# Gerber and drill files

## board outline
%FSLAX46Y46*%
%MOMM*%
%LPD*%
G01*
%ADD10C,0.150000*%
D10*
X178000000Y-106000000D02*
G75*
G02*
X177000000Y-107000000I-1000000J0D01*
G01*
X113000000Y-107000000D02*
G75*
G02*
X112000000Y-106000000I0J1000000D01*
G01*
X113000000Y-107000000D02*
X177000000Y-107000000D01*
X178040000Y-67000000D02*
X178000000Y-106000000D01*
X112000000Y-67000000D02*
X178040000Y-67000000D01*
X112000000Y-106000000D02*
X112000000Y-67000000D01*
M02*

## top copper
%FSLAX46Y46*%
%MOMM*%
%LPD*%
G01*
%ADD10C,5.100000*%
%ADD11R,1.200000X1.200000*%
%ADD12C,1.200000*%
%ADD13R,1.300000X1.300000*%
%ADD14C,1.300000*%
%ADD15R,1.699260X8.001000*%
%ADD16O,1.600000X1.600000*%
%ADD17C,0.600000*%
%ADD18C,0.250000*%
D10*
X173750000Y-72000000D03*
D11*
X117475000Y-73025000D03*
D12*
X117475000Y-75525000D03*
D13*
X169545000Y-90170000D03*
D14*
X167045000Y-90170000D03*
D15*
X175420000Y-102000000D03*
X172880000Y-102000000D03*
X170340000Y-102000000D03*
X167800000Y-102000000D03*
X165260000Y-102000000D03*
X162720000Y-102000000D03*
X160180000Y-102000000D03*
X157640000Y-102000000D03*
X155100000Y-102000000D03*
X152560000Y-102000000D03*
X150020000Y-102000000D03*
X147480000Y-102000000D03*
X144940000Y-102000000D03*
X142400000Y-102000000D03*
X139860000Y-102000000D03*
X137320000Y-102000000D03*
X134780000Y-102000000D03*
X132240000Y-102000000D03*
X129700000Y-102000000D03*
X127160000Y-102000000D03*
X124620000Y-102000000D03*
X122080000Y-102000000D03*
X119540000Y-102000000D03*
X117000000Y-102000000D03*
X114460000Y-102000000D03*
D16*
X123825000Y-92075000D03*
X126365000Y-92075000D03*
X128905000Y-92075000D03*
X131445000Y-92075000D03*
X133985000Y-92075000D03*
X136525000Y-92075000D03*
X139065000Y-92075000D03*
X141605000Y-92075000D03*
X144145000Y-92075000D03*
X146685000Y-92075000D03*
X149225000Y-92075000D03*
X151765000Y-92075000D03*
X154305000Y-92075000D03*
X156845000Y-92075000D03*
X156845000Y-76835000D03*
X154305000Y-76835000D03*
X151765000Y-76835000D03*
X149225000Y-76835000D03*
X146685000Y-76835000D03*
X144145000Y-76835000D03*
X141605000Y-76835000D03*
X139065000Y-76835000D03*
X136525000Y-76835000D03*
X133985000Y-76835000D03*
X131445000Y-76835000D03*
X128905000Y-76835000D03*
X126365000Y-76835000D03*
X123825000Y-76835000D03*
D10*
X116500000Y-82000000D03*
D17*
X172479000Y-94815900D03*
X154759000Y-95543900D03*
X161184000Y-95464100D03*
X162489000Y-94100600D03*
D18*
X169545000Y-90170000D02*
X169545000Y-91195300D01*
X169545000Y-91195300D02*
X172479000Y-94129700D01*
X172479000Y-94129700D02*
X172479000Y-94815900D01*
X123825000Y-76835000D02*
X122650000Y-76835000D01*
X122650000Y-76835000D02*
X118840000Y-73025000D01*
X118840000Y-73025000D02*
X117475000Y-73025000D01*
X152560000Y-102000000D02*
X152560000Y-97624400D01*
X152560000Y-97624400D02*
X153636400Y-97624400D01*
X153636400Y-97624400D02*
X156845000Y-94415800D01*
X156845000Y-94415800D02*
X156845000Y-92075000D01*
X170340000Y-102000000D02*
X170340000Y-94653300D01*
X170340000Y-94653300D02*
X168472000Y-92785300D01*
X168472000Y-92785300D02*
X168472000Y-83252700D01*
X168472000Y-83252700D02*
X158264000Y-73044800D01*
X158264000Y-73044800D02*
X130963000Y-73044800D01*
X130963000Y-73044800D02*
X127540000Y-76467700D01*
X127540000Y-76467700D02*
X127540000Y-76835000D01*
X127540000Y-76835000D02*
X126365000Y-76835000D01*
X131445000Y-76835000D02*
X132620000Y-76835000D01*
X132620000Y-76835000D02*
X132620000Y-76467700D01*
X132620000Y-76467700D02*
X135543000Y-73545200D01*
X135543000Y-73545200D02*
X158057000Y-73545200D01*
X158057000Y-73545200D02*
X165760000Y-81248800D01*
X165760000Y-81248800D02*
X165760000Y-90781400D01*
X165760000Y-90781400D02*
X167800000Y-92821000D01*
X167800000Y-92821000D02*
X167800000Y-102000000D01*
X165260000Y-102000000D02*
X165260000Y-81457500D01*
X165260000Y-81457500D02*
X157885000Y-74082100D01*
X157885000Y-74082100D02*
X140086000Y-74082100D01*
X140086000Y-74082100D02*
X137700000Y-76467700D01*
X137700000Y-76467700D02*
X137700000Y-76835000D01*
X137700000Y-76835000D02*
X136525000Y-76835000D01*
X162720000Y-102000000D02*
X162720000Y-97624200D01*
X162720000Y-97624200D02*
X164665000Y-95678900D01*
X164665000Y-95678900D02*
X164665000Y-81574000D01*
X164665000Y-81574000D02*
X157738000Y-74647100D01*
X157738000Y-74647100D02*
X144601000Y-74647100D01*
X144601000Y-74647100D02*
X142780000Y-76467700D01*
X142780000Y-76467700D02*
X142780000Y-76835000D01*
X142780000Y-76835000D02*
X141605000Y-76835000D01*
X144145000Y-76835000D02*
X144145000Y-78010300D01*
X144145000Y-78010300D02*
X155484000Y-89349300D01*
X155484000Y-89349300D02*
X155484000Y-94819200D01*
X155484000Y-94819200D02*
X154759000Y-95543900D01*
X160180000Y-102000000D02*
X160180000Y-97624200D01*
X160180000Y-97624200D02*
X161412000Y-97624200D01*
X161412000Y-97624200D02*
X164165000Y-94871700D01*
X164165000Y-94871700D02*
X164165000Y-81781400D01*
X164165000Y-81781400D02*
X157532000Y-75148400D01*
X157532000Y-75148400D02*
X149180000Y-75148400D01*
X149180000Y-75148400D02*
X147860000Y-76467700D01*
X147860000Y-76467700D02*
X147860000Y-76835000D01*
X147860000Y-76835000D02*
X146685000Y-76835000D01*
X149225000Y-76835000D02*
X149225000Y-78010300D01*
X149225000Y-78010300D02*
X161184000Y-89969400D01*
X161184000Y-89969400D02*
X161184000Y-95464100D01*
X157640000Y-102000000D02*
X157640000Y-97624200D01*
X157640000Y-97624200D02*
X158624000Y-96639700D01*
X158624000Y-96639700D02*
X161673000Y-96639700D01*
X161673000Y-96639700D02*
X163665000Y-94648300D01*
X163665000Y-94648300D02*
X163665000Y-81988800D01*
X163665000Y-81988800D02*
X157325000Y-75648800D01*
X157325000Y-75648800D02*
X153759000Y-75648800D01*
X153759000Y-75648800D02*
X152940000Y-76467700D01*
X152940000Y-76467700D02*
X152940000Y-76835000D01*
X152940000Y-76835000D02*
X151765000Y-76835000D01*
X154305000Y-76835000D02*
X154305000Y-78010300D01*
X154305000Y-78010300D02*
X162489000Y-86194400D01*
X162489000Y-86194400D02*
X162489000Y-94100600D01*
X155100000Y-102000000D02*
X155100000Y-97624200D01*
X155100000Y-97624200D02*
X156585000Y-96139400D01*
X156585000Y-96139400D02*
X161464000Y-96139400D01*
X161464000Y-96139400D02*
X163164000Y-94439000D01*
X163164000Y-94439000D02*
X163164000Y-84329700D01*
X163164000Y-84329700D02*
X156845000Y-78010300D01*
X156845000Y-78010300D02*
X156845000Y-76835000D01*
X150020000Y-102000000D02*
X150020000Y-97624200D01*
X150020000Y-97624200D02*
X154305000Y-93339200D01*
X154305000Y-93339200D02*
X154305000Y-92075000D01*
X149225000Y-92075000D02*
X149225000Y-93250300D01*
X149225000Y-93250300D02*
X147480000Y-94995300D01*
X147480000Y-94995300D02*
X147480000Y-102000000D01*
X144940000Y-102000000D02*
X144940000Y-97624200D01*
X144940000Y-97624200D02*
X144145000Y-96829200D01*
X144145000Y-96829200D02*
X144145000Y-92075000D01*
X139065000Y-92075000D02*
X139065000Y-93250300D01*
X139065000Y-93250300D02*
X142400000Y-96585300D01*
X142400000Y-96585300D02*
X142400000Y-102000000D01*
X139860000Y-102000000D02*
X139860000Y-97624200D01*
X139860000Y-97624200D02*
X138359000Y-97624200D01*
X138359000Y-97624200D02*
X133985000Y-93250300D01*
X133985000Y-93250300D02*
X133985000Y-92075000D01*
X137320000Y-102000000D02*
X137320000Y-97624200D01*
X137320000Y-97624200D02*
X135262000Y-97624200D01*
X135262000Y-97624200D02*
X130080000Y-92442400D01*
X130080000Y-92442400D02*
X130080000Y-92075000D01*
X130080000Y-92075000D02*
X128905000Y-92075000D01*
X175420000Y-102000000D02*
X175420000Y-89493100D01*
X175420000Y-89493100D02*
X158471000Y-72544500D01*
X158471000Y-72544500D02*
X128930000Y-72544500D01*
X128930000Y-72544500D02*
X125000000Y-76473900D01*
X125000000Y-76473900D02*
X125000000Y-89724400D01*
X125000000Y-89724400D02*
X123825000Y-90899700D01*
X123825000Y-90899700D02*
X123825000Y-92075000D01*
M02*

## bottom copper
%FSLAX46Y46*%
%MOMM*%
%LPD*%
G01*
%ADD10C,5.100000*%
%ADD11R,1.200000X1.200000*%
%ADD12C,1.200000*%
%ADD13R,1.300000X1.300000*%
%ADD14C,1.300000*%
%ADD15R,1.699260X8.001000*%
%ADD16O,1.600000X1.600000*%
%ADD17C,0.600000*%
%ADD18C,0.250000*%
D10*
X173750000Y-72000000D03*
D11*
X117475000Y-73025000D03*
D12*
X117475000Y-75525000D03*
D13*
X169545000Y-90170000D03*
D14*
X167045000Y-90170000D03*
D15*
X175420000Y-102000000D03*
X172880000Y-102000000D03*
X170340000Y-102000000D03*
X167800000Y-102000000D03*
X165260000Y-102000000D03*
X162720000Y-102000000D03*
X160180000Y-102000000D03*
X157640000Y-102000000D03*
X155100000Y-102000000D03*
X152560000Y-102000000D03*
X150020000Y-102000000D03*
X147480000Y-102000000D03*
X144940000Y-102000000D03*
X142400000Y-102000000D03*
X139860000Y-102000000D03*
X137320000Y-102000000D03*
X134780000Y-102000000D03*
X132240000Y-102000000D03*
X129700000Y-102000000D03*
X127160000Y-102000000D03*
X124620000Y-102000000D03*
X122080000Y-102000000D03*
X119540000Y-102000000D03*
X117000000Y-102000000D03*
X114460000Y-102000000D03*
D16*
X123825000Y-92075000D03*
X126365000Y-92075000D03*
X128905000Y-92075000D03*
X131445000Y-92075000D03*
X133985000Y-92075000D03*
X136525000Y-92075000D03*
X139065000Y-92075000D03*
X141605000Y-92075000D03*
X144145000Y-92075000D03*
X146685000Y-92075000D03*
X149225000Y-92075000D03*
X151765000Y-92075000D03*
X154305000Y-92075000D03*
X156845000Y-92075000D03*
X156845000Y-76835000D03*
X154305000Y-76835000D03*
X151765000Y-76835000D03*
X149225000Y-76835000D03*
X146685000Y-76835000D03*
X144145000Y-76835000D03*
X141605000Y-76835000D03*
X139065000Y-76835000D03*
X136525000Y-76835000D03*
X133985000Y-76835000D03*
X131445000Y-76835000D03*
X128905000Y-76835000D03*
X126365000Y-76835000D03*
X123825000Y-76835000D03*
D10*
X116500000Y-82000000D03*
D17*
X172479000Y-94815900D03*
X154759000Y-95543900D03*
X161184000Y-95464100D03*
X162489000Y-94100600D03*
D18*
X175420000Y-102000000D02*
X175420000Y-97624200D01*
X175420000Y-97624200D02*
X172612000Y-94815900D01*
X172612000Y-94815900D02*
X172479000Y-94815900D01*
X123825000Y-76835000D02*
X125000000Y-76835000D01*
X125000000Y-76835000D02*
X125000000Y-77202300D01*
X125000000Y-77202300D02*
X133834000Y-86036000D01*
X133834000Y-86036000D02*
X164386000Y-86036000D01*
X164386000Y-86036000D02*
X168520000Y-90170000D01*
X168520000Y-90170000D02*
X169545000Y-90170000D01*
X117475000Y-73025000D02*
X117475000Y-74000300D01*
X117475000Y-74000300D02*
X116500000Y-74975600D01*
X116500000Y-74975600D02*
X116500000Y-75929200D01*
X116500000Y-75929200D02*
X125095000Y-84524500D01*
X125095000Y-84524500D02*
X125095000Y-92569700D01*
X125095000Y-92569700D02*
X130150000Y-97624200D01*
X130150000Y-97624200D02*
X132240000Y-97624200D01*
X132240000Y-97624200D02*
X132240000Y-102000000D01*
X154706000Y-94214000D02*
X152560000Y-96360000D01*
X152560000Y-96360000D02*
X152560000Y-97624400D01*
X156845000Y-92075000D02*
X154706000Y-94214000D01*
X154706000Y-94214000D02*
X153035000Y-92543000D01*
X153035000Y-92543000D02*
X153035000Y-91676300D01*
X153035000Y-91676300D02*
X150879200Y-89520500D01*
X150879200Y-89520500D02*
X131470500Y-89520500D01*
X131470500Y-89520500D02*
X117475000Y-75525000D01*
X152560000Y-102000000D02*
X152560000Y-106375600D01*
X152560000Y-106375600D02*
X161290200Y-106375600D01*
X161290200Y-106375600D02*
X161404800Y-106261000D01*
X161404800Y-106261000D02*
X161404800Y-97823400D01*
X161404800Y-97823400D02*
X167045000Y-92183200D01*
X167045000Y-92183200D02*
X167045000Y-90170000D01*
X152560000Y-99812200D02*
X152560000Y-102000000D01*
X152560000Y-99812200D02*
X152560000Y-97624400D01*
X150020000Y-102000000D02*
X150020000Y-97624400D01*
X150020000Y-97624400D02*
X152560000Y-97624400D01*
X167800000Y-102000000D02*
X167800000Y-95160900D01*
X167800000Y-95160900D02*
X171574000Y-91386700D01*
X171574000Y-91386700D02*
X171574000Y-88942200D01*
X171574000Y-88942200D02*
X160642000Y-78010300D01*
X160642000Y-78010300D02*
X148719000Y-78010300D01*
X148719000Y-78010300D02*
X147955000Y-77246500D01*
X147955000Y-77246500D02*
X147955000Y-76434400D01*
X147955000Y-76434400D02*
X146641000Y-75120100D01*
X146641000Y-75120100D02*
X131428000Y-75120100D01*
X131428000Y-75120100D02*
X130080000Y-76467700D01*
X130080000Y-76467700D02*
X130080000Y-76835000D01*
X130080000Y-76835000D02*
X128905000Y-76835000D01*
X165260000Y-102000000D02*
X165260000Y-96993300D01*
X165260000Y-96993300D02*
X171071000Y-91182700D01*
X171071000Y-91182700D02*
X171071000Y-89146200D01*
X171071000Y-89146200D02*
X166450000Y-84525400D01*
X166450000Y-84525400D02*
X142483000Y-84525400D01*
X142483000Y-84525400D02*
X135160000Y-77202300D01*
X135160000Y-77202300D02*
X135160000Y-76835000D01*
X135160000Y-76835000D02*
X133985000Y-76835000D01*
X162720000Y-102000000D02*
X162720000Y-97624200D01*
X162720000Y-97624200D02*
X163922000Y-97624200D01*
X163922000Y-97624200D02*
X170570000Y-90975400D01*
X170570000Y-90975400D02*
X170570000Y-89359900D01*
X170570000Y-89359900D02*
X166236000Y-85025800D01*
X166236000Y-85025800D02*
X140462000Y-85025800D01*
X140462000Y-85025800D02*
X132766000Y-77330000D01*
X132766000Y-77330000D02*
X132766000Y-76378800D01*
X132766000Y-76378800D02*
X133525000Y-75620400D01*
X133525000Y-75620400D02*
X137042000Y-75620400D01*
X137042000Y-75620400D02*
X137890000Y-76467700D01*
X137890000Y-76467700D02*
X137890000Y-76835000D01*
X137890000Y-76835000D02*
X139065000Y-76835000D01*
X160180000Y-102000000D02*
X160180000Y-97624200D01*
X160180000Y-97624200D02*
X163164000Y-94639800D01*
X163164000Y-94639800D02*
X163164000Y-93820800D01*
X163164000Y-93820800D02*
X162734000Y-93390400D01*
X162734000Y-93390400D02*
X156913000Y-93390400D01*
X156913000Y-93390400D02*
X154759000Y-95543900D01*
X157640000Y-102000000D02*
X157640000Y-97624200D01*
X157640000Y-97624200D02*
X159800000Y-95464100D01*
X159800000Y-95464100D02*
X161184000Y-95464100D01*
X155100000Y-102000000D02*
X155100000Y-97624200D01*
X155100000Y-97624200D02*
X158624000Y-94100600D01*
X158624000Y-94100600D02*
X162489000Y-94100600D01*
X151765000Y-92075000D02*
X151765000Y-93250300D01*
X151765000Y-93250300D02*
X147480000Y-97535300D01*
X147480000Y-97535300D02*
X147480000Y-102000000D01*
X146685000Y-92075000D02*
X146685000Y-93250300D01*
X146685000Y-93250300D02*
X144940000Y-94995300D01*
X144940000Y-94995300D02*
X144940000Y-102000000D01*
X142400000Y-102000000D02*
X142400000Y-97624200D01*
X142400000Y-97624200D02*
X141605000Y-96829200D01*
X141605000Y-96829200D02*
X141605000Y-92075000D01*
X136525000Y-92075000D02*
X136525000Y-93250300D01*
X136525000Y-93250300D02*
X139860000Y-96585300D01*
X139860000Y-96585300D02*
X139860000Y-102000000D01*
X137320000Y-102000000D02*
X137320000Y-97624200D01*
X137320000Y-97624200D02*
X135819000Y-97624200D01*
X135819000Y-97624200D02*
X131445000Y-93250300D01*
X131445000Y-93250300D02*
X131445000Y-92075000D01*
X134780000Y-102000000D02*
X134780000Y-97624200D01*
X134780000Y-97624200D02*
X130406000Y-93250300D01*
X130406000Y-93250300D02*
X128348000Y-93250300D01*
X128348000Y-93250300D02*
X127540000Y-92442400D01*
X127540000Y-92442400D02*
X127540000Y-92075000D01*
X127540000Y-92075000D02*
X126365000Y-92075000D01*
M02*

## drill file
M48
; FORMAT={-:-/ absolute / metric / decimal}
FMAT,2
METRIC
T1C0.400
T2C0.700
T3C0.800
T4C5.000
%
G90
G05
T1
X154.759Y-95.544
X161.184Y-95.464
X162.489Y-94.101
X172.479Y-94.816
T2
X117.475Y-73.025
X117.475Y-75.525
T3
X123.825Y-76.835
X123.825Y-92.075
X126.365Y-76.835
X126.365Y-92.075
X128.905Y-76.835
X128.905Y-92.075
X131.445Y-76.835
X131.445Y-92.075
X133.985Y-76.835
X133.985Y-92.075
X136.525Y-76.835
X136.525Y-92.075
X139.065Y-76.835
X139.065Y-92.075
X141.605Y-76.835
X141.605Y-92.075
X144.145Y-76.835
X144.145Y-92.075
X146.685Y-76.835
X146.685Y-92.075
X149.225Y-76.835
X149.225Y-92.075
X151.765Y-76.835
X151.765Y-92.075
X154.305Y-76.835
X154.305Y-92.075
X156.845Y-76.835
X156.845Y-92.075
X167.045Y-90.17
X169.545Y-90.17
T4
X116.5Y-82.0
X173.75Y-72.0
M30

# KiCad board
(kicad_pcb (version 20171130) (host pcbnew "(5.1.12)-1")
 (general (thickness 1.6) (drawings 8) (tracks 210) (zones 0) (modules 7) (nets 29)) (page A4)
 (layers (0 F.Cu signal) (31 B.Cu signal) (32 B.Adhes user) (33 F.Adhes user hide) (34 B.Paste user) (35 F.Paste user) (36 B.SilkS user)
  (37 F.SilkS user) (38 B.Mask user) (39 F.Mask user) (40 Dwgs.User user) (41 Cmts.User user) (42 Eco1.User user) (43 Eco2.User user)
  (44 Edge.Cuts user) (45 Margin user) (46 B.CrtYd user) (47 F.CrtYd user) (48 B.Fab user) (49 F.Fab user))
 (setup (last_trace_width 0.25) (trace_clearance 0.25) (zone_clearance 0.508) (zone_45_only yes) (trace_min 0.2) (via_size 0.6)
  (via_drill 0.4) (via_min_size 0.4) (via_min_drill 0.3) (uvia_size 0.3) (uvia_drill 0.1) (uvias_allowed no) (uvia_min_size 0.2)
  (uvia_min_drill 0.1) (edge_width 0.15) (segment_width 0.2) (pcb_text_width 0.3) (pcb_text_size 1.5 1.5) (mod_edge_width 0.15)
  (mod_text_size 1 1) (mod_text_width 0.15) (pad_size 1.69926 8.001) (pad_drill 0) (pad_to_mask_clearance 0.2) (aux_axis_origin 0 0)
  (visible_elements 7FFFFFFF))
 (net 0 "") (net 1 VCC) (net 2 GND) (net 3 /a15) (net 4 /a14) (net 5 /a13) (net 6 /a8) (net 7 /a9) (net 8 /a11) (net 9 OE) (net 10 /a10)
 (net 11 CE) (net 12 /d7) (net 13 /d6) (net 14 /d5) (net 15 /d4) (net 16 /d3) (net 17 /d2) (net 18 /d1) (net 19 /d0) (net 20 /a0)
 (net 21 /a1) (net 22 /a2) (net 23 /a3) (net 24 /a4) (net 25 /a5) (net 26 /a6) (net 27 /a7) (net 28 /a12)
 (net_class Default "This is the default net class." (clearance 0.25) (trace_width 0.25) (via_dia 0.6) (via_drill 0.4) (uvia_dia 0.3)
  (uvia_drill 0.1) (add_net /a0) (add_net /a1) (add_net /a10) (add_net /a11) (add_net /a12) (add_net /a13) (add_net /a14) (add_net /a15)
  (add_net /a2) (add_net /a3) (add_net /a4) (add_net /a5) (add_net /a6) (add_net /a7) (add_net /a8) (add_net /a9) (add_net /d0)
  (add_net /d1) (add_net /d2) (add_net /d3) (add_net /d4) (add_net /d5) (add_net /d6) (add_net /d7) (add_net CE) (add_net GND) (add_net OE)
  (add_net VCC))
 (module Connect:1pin (layer F.Cu) (at 173.75 72)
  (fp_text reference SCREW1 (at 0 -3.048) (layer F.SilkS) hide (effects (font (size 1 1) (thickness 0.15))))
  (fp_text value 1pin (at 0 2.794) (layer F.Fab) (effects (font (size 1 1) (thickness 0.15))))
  (pad "" np_thru_hole circle (at 0 0) (size 5.1 5.1) (drill 5) (layers *.Cu)))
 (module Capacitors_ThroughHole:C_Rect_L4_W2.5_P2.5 (layer F.Cu) (at 117.475 73.025 270)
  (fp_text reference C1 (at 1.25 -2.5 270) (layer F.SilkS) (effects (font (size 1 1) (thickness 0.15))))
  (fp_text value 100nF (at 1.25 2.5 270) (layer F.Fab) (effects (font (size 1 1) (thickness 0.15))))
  (pad 1 thru_hole rect (at 0 0 270) (size 1.2 1.2) (drill 0.7) (layers *.Cu *.Mask F.SilkS) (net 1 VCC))
  (pad 2 thru_hole circle (at 2.5 0 270) (size 1.2 1.2) (drill 0.7) (layers *.Cu *.Mask F.SilkS) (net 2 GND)))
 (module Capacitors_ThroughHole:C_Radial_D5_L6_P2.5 (layer F.Cu) (at 169.545 90.17 180)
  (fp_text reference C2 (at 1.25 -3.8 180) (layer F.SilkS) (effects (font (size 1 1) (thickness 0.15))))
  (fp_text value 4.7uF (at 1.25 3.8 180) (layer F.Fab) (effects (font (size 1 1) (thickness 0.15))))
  (pad 1 thru_hole rect (at 0 0 180) (size 1.3 1.3) (drill 0.8) (layers *.Cu *.Mask F.SilkS) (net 1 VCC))
  (pad 2 thru_hole circle (at 2.5 0 180) (size 1.3 1.3) (drill 0.8) (layers *.Cu *.Mask F.SilkS) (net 2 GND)))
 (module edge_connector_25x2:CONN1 (layer F.Cu) (at 144.94 107.08)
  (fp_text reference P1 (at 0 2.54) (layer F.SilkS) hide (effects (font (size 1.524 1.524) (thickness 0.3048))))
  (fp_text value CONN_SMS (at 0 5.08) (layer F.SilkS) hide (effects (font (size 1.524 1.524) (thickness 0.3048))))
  (pad 1 connect rect (at 30.48 -5.08) (size 1.69926 8.001) (layers B.Cu B.Mask) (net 1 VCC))
  (pad 2 connect rect (at 30.48 -5.08) (size 1.69926 8.001) (layers F.Cu F.Mask) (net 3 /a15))
  (pad 3 connect rect (at 27.94 -5.08) (size 1.69926 8.001) (layers B.Cu B.Mask))
  (pad 4 connect rect (at 27.94 -5.08) (size 1.69926 8.001) (layers F.Cu F.Mask))
  (pad 5 connect rect (at 25.4 -5.08) (size 1.69926 8.001) (layers B.Cu B.Mask))
  (pad 6 connect rect (at 25.4 -5.08) (size 1.69926 8.001) (layers F.Cu F.Mask) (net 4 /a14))
  (pad 7 connect rect (at 22.86 -5.08) (size 1.69926 8.001) (layers B.Cu B.Mask) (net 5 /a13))
  (pad 8 connect rect (at 22.86 -5.08) (size 1.69926 8.001) (layers F.Cu F.Mask) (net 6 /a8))
  (pad 9 connect rect (at 20.32 -5.08) (size 1.69926 8.001) (layers B.Cu B.Mask) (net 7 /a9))
  (pad 10 connect rect (at 20.32 -5.08) (size 1.69926 8.001) (layers F.Cu F.Mask) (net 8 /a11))
  (pad 11 connect rect (at 17.78 -5.08) (size 1.69926 8.001) (layers B.Cu B.Mask) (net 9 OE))
  (pad 12 connect rect (at 17.78 -5.08) (size 1.69926 8.001) (layers F.Cu F.Mask) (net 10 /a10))
  (pad 13 connect rect (at 15.24 -5.08) (size 1.69926 8.001) (layers B.Cu B.Mask) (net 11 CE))
  (pad 14 connect rect (at 15.24 -5.08) (size 1.69926 8.001) (layers F.Cu F.Mask) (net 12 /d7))
  (pad 15 connect rect (at 12.7 -5.08) (size 1.69926 8.001) (layers B.Cu B.Mask) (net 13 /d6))
  (pad 16 connect rect (at 12.7 -5.08) (size 1.69926 8.001) (layers F.Cu F.Mask) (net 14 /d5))
  (pad 17 connect rect (at 10.16 -5.08) (size 1.69926 8.001) (layers B.Cu B.Mask) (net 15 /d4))
  (pad 18 connect rect (at 10.16 -5.08) (size 1.69926 8.001) (layers F.Cu F.Mask) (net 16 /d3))
  (pad 19 connect rect (at 7.62 -5.08) (size 1.69926 8.001) (layers B.Cu B.Mask) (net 2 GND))
  (pad 20 connect rect (at 7.62 -5.08) (size 1.69926 8.001) (layers F.Cu F.Mask) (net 2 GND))
  (pad 21 connect rect (at 5.08 -5.08) (size 1.69926 8.001) (layers B.Cu B.Mask) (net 2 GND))
  (pad 22 connect rect (at 5.08 -5.08) (size 1.69926 8.001) (layers F.Cu F.Mask) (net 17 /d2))
  (pad 23 connect rect (at 2.54 -5.08) (size 1.69926 8.001) (layers B.Cu B.Mask) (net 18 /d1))
  (pad 24 connect rect (at 2.54 -5.08) (size 1.69926 8.001) (layers F.Cu F.Mask) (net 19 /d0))
  (pad 25 connect rect (at 0 -5.08) (size 1.69926 8.001) (layers B.Cu B.Mask) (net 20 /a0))
  (pad 26 connect rect (at 0 -5.08) (size 1.69926 8.001) (layers F.Cu F.Mask) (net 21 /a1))
  (pad 27 connect rect (at -2.54 -5.08) (size 1.69926 8.001) (layers B.Cu B.Mask) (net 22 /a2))
  (pad 28 connect rect (at -2.54 -5.08) (size 1.69926 8.001) (layers F.Cu F.Mask) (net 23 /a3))
  (pad 29 connect rect (at -5.08 -5.08) (size 1.69926 8.001) (layers B.Cu B.Mask) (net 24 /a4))
  (pad 30 connect rect (at -5.08 -5.08) (size 1.69926 8.001) (layers F.Cu F.Mask) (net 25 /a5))
  (pad 31 connect rect (at -7.62 -5.08) (size 1.69926 8.001) (layers B.Cu B.Mask) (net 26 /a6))
  (pad 32 connect rect (at -7.62 -5.08) (size 1.69926 8.001) (layers F.Cu F.Mask) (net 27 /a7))
  (pad 33 connect rect (at -10.16 -5.08) (size 1.69926 8.001) (layers B.Cu B.Mask) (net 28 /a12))
  (pad 34 connect rect (at -10.16 -5.08) (size 1.69926 8.001) (layers F.Cu F.Mask))
  (pad 35 connect rect (at -12.7 -5.08) (size 1.69926 8.001) (layers B.Cu B.Mask) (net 1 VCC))
  (pad 36 connect rect (at -12.7 -5.08) (size 1.69926 8.001) (layers F.Cu F.Mask))
  (pad 37 connect rect (at -15.24 -5.08) (size 1.69926 8.001) (layers B.Cu B.Mask))
  (pad 38 connect rect (at -15.24 -5.08) (size 1.69926 8.001) (layers F.Cu F.Mask))
  (pad 39 connect rect (at -17.78 -5.08) (size 1.69926 8.001) (layers B.Cu B.Mask))
  (pad 40 connect rect (at -17.78 -5.08) (size 1.69926 8.001) (layers F.Cu F.Mask))
  (pad 41 connect rect (at -20.32 -5.08) (size 1.69926 8.001) (layers B.Cu B.Mask))
  (pad 42 connect rect (at -20.32 -5.08) (size 1.69926 8.001) (layers F.Cu F.Mask))
  (pad 43 connect rect (at -22.86 -5.08) (size 1.69926 8.001) (layers B.Cu B.Mask))
  (pad 44 connect rect (at -22.86 -5.08) (size 1.69926 8.001) (layers F.Cu F.Mask))
  (pad 45 connect rect (at -25.4 -5.08) (size 1.69926 8.001) (layers B.Cu B.Mask))
  (pad 46 connect rect (at -25.4 -5.08) (size 1.69926 8.001) (layers F.Cu F.Mask))
  (pad 47 connect rect (at -27.94 -5.08) (size 1.69926 8.001) (layers B.Cu B.Mask))
  (pad 48 connect rect (at -27.94 -5.08) (size 1.69926 8.001) (layers F.Cu F.Mask))
  (pad 49 connect rect (at -30.48 -5.08) (size 1.69926 8.001) (layers B.Cu B.Mask))
  (pad 50 connect rect (at -30.48 -5.08) (size 1.69926 8.001) (layers F.Cu F.Mask)))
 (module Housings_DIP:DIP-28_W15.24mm (layer F.Cu) (at 123.825 92.075 90)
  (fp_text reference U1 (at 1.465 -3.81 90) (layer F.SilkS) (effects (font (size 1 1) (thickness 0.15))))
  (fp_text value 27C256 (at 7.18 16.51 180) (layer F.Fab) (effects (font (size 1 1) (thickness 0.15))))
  (pad 1 thru_hole oval (at 0 0 90) (size 1.6 1.6) (drill 0.8) (layers *.Cu *.Mask F.SilkS) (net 3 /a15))
  (pad 2 thru_hole oval (at 0 2.54 90) (size 1.6 1.6) (drill 0.8) (layers *.Cu *.Mask F.SilkS) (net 28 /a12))
  (pad 3 thru_hole oval (at 0 5.08 90) (size 1.6 1.6) (drill 0.8) (layers *.Cu *.Mask F.SilkS) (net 27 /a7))
  (pad 4 thru_hole oval (at 0 7.62 90) (size 1.6 1.6) (drill 0.8) (layers *.Cu *.Mask F.SilkS) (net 26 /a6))
  (pad 5 thru_hole oval (at 0 10.16 90) (size 1.6 1.6) (drill 0.8) (layers *.Cu *.Mask F.SilkS) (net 25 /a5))
  (pad 6 thru_hole oval (at 0 12.7 90) (size 1.6 1.6) (drill 0.8) (layers *.Cu *.Mask F.SilkS) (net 24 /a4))
  (pad 7 thru_hole oval (at 0 15.24 90) (size 1.6 1.6) (drill 0.8) (layers *.Cu *.Mask F.SilkS) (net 23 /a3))
  (pad 8 thru_hole oval (at 0 17.78 90) (size 1.6 1.6) (drill 0.8) (layers *.Cu *.Mask F.SilkS) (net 22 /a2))
  (pad 9 thru_hole oval (at 0 20.32 90) (size 1.6 1.6) (drill 0.8) (layers *.Cu *.Mask F.SilkS) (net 21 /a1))
  (pad 10 thru_hole oval (at 0 22.86 90) (size 1.6 1.6) (drill 0.8) (layers *.Cu *.Mask F.SilkS) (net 20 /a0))
  (pad 11 thru_hole oval (at 0 25.4 90) (size 1.6 1.6) (drill 0.8) (layers *.Cu *.Mask F.SilkS) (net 19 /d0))
  (pad 12 thru_hole oval (at 0 27.94 90) (size 1.6 1.6) (drill 0.8) (layers *.Cu *.Mask F.SilkS) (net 18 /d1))
  (pad 13 thru_hole oval (at 0 30.48 90) (size 1.6 1.6) (drill 0.8) (layers *.Cu *.Mask F.SilkS) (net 17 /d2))
  (pad 14 thru_hole oval (at 0 33.02 90) (size 1.6 1.6) (drill 0.8) (layers *.Cu *.Mask F.SilkS) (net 2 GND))
  (pad 15 thru_hole oval (at 15.24 33.02 90) (size 1.6 1.6) (drill 0.8) (layers *.Cu *.Mask F.SilkS) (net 16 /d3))
  (pad 16 thru_hole oval (at 15.24 30.48 90) (size 1.6 1.6) (drill 0.8) (layers *.Cu *.Mask F.SilkS) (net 15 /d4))
  (pad 17 thru_hole oval (at 15.24 27.94 90) (size 1.6 1.6) (drill 0.8) (layers *.Cu *.Mask F.SilkS) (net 14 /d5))
  (pad 18 thru_hole oval (at 15.24 25.4 90) (size 1.6 1.6) (drill 0.8) (layers *.Cu *.Mask F.SilkS) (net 13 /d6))
  (pad 19 thru_hole oval (at 15.24 22.86 90) (size 1.6 1.6) (drill 0.8) (layers *.Cu *.Mask F.SilkS) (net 12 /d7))
  (pad 20 thru_hole oval (at 15.24 20.32 90) (size 1.6 1.6) (drill 0.8) (layers *.Cu *.Mask F.SilkS) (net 11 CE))
  (pad 21 thru_hole oval (at 15.24 17.78 90) (size 1.6 1.6) (drill 0.8) (layers *.Cu *.Mask F.SilkS) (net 10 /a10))
  (pad 22 thru_hole oval (at 15.24 15.24 90) (size 1.6 1.6) (drill 0.8) (layers *.Cu *.Mask F.SilkS) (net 9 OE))
  (pad 23 thru_hole oval (at 15.24 12.7 90) (size 1.6 1.6) (drill 0.8) (layers *.Cu *.Mask F.SilkS) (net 8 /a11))
  (pad 24 thru_hole oval (at 15.24 10.16 90) (size 1.6 1.6) (drill 0.8) (layers *.Cu *.Mask F.SilkS) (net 7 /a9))
  (pad 25 thru_hole oval (at 15.24 7.62 90) (size 1.6 1.6) (drill 0.8) (layers *.Cu *.Mask F.SilkS) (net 6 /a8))
  (pad 26 thru_hole oval (at 15.24 5.08 90) (size 1.6 1.6) (drill 0.8) (layers *.Cu *.Mask F.SilkS) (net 5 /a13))
  (pad 27 thru_hole oval (at 15.24 2.54 90) (size 1.6 1.6) (drill 0.8) (layers *.Cu *.Mask F.SilkS) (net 4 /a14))
  (pad 28 thru_hole oval (at 15.24 0 90) (size 1.6 1.6) (drill 0.8) (layers *.Cu *.Mask F.SilkS) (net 1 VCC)))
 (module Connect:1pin (layer F.Cu) (at 116.5 82)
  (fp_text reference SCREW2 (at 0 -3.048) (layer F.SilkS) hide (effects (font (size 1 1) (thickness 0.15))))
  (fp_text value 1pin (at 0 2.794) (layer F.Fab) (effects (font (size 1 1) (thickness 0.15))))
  (pad "" np_thru_hole circle (at 0 0) (size 5.1 5.1) (drill 5) (layers *.Cu)))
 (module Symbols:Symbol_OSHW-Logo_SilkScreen (layer F.Cu) (at 166 71)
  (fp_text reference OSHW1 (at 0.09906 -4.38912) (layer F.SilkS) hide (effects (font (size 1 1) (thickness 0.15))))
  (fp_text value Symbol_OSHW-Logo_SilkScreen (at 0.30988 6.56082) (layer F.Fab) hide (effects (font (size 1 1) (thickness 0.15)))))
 (gr_arc (start 177 106) (end 178 106) (angle 90) (layer Edge.Cuts) (width 0.15))
 (gr_arc (start 113 106) (end 113 107) (angle 90) (layer Edge.Cuts) (width 0.15))
 (gr_line (start 113 107) (end 177 107) (layer Edge.Cuts) (width 0.15))
 (gr_line (start 178.04 67) (end 178 106) (angle 90) (layer Edge.Cuts) (width 0.15))
 (gr_line (start 112 67) (end 178.04 67) (angle 90) (layer Edge.Cuts) (width 0.15))
 (gr_line (start 112 106) (end 112 67) (angle 90) (layer Edge.Cuts) (width 0.15))
 (segment (start 169.545 90.17) (end 169.545 91.1953) (width 0.25) (layer F.Cu) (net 1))
 (segment (start 169.545 91.1953) (end 172.479 94.1297) (width 0.25) (layer F.Cu) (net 1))
 (segment (start 172.479 94.1297) (end 172.479 94.8159) (width 0.25) (layer F.Cu) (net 1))
 (segment (start 175.42 102) (end 175.42 97.6242) (width 0.25) (layer B.Cu) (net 1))
 (segment (start 175.42 97.6242) (end 172.612 94.8159) (width 0.25) (layer B.Cu) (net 1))
 (segment (start 172.612 94.8159) (end 172.479 94.8159) (width 0.25) (layer B.Cu) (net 1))
 (segment (start 123.825 76.835) (end 125 76.835) (width 0.25) (layer B.Cu) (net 1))
 (segment (start 125 76.835) (end 125 77.2023) (width 0.25) (layer B.Cu) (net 1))
 (segment (start 125 77.2023) (end 133.834 86.036) (width 0.25) (layer B.Cu) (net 1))
 (segment (start 133.834 86.036) (end 164.386 86.036) (width 0.25) (layer B.Cu) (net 1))
 (segment (start 164.386 86.036) (end 168.52 90.17) (width 0.25) (layer B.Cu) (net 1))
 (segment (start 168.52 90.17) (end 169.545 90.17) (width 0.25) (layer B.Cu) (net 1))
 (segment (start 117.475 73.025) (end 117.475 74.0003) (width 0.25) (layer B.Cu) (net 1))
 (segment (start 117.475 74.0003) (end 116.5 74.9756) (width 0.25) (layer B.Cu) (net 1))
 (segment (start 116.5 74.9756) (end 116.5 75.9292) (width 0.25) (layer B.Cu) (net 1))
 (segment (start 116.5 75.9292) (end 125.095 84.5245) (width 0.25) (layer B.Cu) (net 1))
 (segment (start 125.095 84.5245) (end 125.095 92.5697) (width 0.25) (layer B.Cu) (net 1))
 (segment (start 125.095 92.5697) (end 130.15 97.6242) (width 0.25) (layer B.Cu) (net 1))
 (segment (start 130.15 97.6242) (end 132.24 97.6242) (width 0.25) (layer B.Cu) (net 1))
 (segment (start 132.24 97.6242) (end 132.24 102) (width 0.25) (layer B.Cu) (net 1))
 (segment (start 123.825 76.835) (end 122.65 76.835) (width 0.25) (layer F.Cu) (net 1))
 (segment (start 122.65 76.835) (end 118.84 73.025) (width 0.25) (layer F.Cu) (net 1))
 (segment (start 118.84 73.025) (end 117.475 73.025) (width 0.25) (layer F.Cu) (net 1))
 (via (at 172.479 94.8159) (size 0.6) (layers F.Cu B.Cu) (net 1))
 (segment (start 154.706 94.214) (end 152.56 96.36) (width 0.25) (layer B.Cu) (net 2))
 (segment (start 152.56 96.36) (end 152.56 97.6244) (width 0.25) (layer B.Cu) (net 2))
 (segment (start 156.845 92.075) (end 154.706 94.214) (width 0.25) (layer B.Cu) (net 2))
 (segment (start 154.706 94.214) (end 153.035 92.543) (width 0.25) (layer B.Cu) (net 2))
 (segment (start 153.035 92.543) (end 153.035 91.6763) (width 0.25) (layer B.Cu) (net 2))
 (segment (start 153.035 91.6763) (end 150.8792 89.5205) (width 0.25) (layer B.Cu) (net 2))
 (segment (start 150.8792 89.5205) (end 131.4705 89.5205) (width 0.25) (layer B.Cu) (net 2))
 (segment (start 131.4705 89.5205) (end 117.475 75.525) (width 0.25) (layer B.Cu) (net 2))
 (segment (start 152.56 102) (end 152.56 106.3756) (width 0.25) (layer B.Cu) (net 2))
 (segment (start 152.56 106.3756) (end 161.2902 106.3756) (width 0.25) (layer B.Cu) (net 2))
 (segment (start 161.2902 106.3756) (end 161.4048 106.261) (width 0.25) (layer B.Cu) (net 2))
 (segment (start 161.4048 106.261) (end 161.4048 97.8234) (width 0.25) (layer B.Cu) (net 2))
 (segment (start 161.4048 97.8234) (end 167.045 92.1832) (width 0.25) (layer B.Cu) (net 2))
 (segment (start 167.045 92.1832) (end 167.045 90.17) (width 0.25) (layer B.Cu) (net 2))
 (segment (start 152.56 99.8122) (end 152.56 102) (width 0.25) (layer B.Cu) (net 2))
 (segment (start 152.56 99.8122) (end 152.56 97.6244) (width 0.25) (layer B.Cu) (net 2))
 (segment (start 152.56 102) (end 152.56 97.6244) (width 0.25) (layer F.Cu) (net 2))
 (segment (start 152.56 97.6244) (end 153.6364 97.6244) (width 0.25) (layer F.Cu) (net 2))
 (segment (start 153.6364 97.6244) (end 156.845 94.4158) (width 0.25) (layer F.Cu) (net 2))
 (segment (start 156.845 94.4158) (end 156.845 92.075) (width 0.25) (layer F.Cu) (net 2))
 (segment (start 150.02 102) (end 150.02 97.6244) (width 0.25) (layer B.Cu) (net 2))
 (segment (start 150.02 97.6244) (end 152.56 97.6244) (width 0.25) (layer B.Cu) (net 2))
 (segment (start 170.34 102) (end 170.34 94.6533) (width 0.25) (layer F.Cu) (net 4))
 (segment (start 170.34 94.6533) (end 168.472 92.7853) (width 0.25) (layer F.Cu) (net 4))
 (segment (start 168.472 92.7853) (end 168.472 83.2527) (width 0.25) (layer F.Cu) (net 4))
 (segment (start 168.472 83.2527) (end 158.264 73.0448) (width 0.25) (layer F.Cu) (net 4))
 (segment (start 158.264 73.0448) (end 130.963 73.0448) (width 0.25) (layer F.Cu) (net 4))
 (segment (start 130.963 73.0448) (end 127.54 76.4677) (width 0.25) (layer F.Cu) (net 4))
 (segment (start 127.54 76.4677) (end 127.54 76.835) (width 0.25) (layer F.Cu) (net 4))
 (segment (start 127.54 76.835) (end 126.365 76.835) (width 0.25) (layer F.Cu) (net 4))
 (segment (start 167.8 102) (end 167.8 95.1609) (width 0.25) (layer B.Cu) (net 5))
 (segment (start 167.8 95.1609) (end 171.574 91.3867) (width 0.25) (layer B.Cu) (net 5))
 (segment (start 171.574 91.3867) (end 171.574 88.9422) (width 0.25) (layer B.Cu) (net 5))
 (segment (start 171.574 88.9422) (end 160.642 78.0103) (width 0.25) (layer B.Cu) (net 5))
 (segment (start 160.642 78.0103) (end 148.719 78.0103) (width 0.25) (layer B.Cu) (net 5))
 (segment (start 148.719 78.0103) (end 147.955 77.2465) (width 0.25) (layer B.Cu) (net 5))
 (segment (start 147.955 77.2465) (end 147.955 76.4344) (width 0.25) (layer B.Cu) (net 5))
 (segment (start 147.955 76.4344) (end 146.641 75.1201) (width 0.25) (layer B.Cu) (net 5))
 (segment (start 146.641 75.1201) (end 131.428 75.1201) (width 0.25) (layer B.Cu) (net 5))
 (segment (start 131.428 75.1201) (end 130.08 76.4677) (width 0.25) (layer B.Cu) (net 5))
 (segment (start 130.08 76.4677) (end 130.08 76.835) (width 0.25) (layer B.Cu) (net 5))
 (segment (start 130.08 76.835) (end 128.905 76.835) (width 0.25) (layer B.Cu) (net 5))
 (segment (start 131.445 76.835) (end 132.62 76.835) (width 0.25) (layer F.Cu) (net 6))
 (segment (start 132.62 76.835) (end 132.62 76.4677) (width 0.25) (layer F.Cu) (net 6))
 (segment (start 132.62 76.4677) (end 135.543 73.5452) (width 0.25) (layer F.Cu) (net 6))
 (segment (start 135.543 73.5452) (end 158.057 73.5452) (width 0.25) (layer F.Cu) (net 6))
 (segment (start 158.057 73.5452) (end 165.76 81.2488) (width 0.25) (layer F.Cu) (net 6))
 (segment (start 165.76 81.2488) (end 165.76 90.7814) (width 0.25) (layer F.Cu) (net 6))
 (segment (start 165.76 90.7814) (end 167.8 92.821) (width 0.25) (layer F.Cu) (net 6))
 (segment (start 167.8 92.821) (end 167.8 102) (width 0.25) (layer F.Cu) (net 6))
 (segment (start 165.26 102) (end 165.26 96.9933) (width 0.25) (layer B.Cu) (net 7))
 (segment (start 165.26 96.9933) (end 171.071 91.1827) (width 0.25) (layer B.Cu) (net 7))
 (segment (start 171.071 91.1827) (end 171.071 89.1462) (width 0.25) (layer B.Cu) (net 7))
 (segment (start 171.071 89.1462) (end 166.45 84.5254) (width 0.25) (layer B.Cu) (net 7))
 (segment (start 166.45 84.5254) (end 142.483 84.5254) (width 0.25) (layer B.Cu) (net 7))
 (segment (start 142.483 84.5254) (end 135.16 77.2023) (width 0.25) (layer B.Cu) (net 7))
 (segment (start 135.16 77.2023) (end 135.16 76.835) (width 0.25) (layer B.Cu) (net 7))
 (segment (start 135.16 76.835) (end 133.985 76.835) (width 0.25) (layer B.Cu) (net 7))
 (segment (start 165.26 102) (end 165.26 81.4575) (width 0.25) (layer F.Cu) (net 8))
 (segment (start 165.26 81.4575) (end 157.885 74.0821) (width 0.25) (layer F.Cu) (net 8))
 (segment (start 157.885 74.0821) (end 140.086 74.0821) (width 0.25) (layer F.Cu) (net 8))
 (segment (start 140.086 74.0821) (end 137.7 76.4677) (width 0.25) (layer F.Cu) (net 8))
 (segment (start 137.7 76.4677) (end 137.7 76.835) (width 0.25) (layer F.Cu) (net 8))
 (segment (start 137.7 76.835) (end 136.525 76.835) (width 0.25) (layer F.Cu) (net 8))
 (segment (start 162.72 102) (end 162.72 97.6242) (width 0.25) (layer B.Cu) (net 9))
 (segment (start 162.72 97.6242) (end 163.922 97.6242) (width 0.25) (layer B.Cu) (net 9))
 (segment (start 163.922 97.6242) (end 170.57 90.9754) (width 0.25) (layer B.Cu) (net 9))
 (segment (start 170.57 90.9754) (end 170.57 89.3599) (width 0.25) (layer B.Cu) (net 9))
 (segment (start 170.57 89.3599) (end 166.236 85.0258) (width 0.25) (layer B.Cu) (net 9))
 (segment (start 166.236 85.0258) (end 140.462 85.0258) (width 0.25) (layer B.Cu) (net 9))
 (segment (start 140.462 85.0258) (end 132.766 77.33) (width 0.25) (layer B.Cu) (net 9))
 (segment (start 132.766 77.33) (end 132.766 76.3788) (width 0.25) (layer B.Cu) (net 9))
 (segment (start 132.766 76.3788) (end 133.525 75.6204) (width 0.25) (layer B.Cu) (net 9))
 (segment (start 133.525 75.6204) (end 137.042 75.6204) (width 0.25) (layer B.Cu) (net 9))
 (segment (start 137.042 75.6204) (end 137.89 76.4677) (width 0.25) (layer B.Cu) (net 9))
 (segment (start 137.89 76.4677) (end 137.89 76.835) (width 0.25) (layer B.Cu) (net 9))
 (segment (start 137.89 76.835) (end 139.065 76.835) (width 0.25) (layer B.Cu) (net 9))
 (segment (start 162.72 102) (end 162.72 97.6242) (width 0.25) (layer F.Cu) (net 10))
 (segment (start 162.72 97.6242) (end 164.665 95.6789) (width 0.25) (layer F.Cu) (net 10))
 (segment (start 164.665 95.6789) (end 164.665 81.574) (width 0.25) (layer F.Cu) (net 10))
 (segment (start 164.665 81.574) (end 157.738 74.6471) (width 0.25) (layer F.Cu) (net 10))
 (segment (start 157.738 74.6471) (end 144.601 74.6471) (width 0.25) (layer F.Cu) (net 10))
 (segment (start 144.601 74.6471) (end 142.78 76.4677) (width 0.25) (layer F.Cu) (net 10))
 (segment (start 142.78 76.4677) (end 142.78 76.835) (width 0.25) (layer F.Cu) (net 10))
 (segment (start 142.78 76.835) (end 141.605 76.835) (width 0.25) (layer F.Cu) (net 10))
 (segment (start 144.145 76.835) (end 144.145 78.0103) (width 0.25) (layer F.Cu) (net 11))
 (segment (start 144.145 78.0103) (end 155.484 89.3493) (width 0.25) (layer F.Cu) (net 11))
 (segment (start 155.484 89.3493) (end 155.484 94.8192) (width 0.25) (layer F.Cu) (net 11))
 (segment (start 155.484 94.8192) (end 154.759 95.5439) (width 0.25) (layer F.Cu) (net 11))
 (segment (start 160.18 102) (end 160.18 97.6242) (width 0.25) (layer B.Cu) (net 11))
 (segment (start 160.18 97.6242) (end 163.164 94.6398) (width 0.25) (layer B.Cu) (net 11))
 (segment (start 163.164 94.6398) (end 163.164 93.8208) (width 0.25) (layer B.Cu) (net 11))
 (segment (start 163.164 93.8208) (end 162.734 93.3904) (width 0.25) (layer B.Cu) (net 11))
 (segment (start 162.734 93.3904) (end 156.913 93.3904) (width 0.25) (layer B.Cu) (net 11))
 (segment (start 156.913 93.3904) (end 154.759 95.5439) (width 0.25) (layer B.Cu) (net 11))
 (via (at 154.759 95.5439) (size 0.6) (layers F.Cu B.Cu) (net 11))
 (segment (start 160.18 102) (end 160.18 97.6242) (width 0.25) (layer F.Cu) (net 12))
 (segment (start 160.18 97.6242) (end 161.412 97.6242) (width 0.25) (layer F.Cu) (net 12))
 (segment (start 161.412 97.6242) (end 164.165 94.8717) (width 0.25) (layer F.Cu) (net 12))
 (segment (start 164.165 94.8717) (end 164.165 81.7814) (width 0.25) (layer F.Cu) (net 12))
 (segment (start 164.165 81.7814) (end 157.532 75.1484) (width 0.25) (layer F.Cu) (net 12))
 (segment (start 157.532 75.1484) (end 149.18 75.1484) (width 0.25) (layer F.Cu) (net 12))
 (segment (start 149.18 75.1484) (end 147.86 76.4677) (width 0.25) (layer F.Cu) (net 12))
 (segment (start 147.86 76.4677) (end 147.86 76.835) (width 0.25) (layer F.Cu) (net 12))
 (segment (start 147.86 76.835) (end 146.685 76.835) (width 0.25) (layer F.Cu) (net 12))
 (segment (start 149.225 76.835) (end 149.225 78.0103) (width 0.25) (layer F.Cu) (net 13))
 (segment (start 149.225 78.0103) (end 161.184 89.9694) (width 0.25) (layer F.Cu) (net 13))
 (segment (start 161.184 89.9694) (end 161.184 95.4641) (width 0.25) (layer F.Cu) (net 13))
 (segment (start 157.64 102) (end 157.64 97.6242) (width 0.25) (layer B.Cu) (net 13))
 (segment (start 157.64 97.6242) (end 159.8 95.4641) (width 0.25) (layer B.Cu) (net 13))
 (segment (start 159.8 95.4641) (end 161.184 95.4641) (width 0.25) (layer B.Cu) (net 13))
 (via (at 161.184 95.4641) (size 0.6) (layers F.Cu B.Cu) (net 13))
 (segment (start 157.64 102) (end 157.64 97.6242) (width 0.25) (layer F.Cu) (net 14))
 (segment (start 157.64 97.6242) (end 158.624 96.6397) (width 0.25) (layer F.Cu) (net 14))
 (segment (start 158.624 96.6397) (end 161.673 96.6397) (width 0.25) (layer F.Cu) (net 14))
 (segment (start 161.673 96.6397) (end 163.665 94.6483) (width 0.25) (layer F.Cu) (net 14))
 (segment (start 163.665 94.6483) (end 163.665 81.9888) (width 0.25) (layer F.Cu) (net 14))
 (segment (start 163.665 81.9888) (end 157.325 75.6488) (width 0.25) (layer F.Cu) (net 14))
 (segment (start 157.325 75.6488) (end 153.759 75.6488) (width 0.25) (layer F.Cu) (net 14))
 (segment (start 153.759 75.6488) (end 152.94 76.4677) (width 0.25) (layer F.Cu) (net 14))
 (segment (start 152.94 76.4677) (end 152.94 76.835) (width 0.25) (layer F.Cu) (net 14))
 (segment (start 152.94 76.835) (end 151.765 76.835) (width 0.25) (layer F.Cu) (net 14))
 (segment (start 155.1 102) (end 155.1 97.6242) (width 0.25) (layer B.Cu) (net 15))
 (segment (start 155.1 97.6242) (end 158.624 94.1006) (width 0.25) (layer B.Cu) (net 15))
 (segment (start 158.624 94.1006) (end 162.489 94.1006) (width 0.25) (layer B.Cu) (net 15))
 (segment (start 154.305 76.835) (end 154.305 78.0103) (width 0.25) (layer F.Cu) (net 15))
 (segment (start 154.305 78.0103) (end 162.489 86.1944) (width 0.25) (layer F.Cu) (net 15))
 (segment (start 162.489 86.1944) (end 162.489 94.1006) (width 0.25) (layer F.Cu) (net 15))
 (via (at 162.489 94.1006) (size 0.6) (layers F.Cu B.Cu) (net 15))
 (segment (start 155.1 102) (end 155.1 97.6242) (width 0.25) (layer F.Cu) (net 16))
 (segment (start 155.1 97.6242) (end 156.585 96.1394) (width 0.25) (layer F.Cu) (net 16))
 (segment (start 156.585 96.1394) (end 161.464 96.1394) (width 0.25) (layer F.Cu) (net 16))
 (segment (start 161.464 96.1394) (end 163.164 94.439) (width 0.25) (layer F.Cu) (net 16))
 (segment (start 163.164 94.439) (end 163.164 84.3297) (width 0.25) (layer F.Cu) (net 16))
 (segment (start 163.164 84.3297) (end 156.845 78.0103) (width 0.25) (layer F.Cu) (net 16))
 (segment (start 156.845 78.0103) (end 156.845 76.835) (width 0.25) (layer F.Cu) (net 16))
 (segment (start 150.02 102) (end 150.02 97.6242) (width 0.25) (layer F.Cu) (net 17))
 (segment (start 150.02 97.6242) (end 154.305 93.3392) (width 0.25) (layer F.Cu) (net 17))
 (segment (start 154.305 93.3392) (end 154.305 92.075) (width 0.25) (layer F.Cu) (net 17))
 (segment (start 151.765 92.075) (end 151.765 93.2503) (width 0.25) (layer B.Cu) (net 18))
 (segment (start 151.765 93.2503) (end 147.48 97.5353) (width 0.25) (layer B.Cu) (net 18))
 (segment (start 147.48 97.5353) (end 147.48 102) (width 0.25) (layer B.Cu) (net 18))
 (segment (start 149.225 92.075) (end 149.225 93.2503) (width 0.25) (layer F.Cu) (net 19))
 (segment (start 149.225 93.2503) (end 147.48 94.9953) (width 0.25) (layer F.Cu) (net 19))
 (segment (start 147.48 94.9953) (end 147.48 102) (width 0.25) (layer F.Cu) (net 19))
 (segment (start 146.685 92.075) (end 146.685 93.2503) (width 0.25) (layer B.Cu) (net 20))
 (segment (start 146.685 93.2503) (end 144.94 94.9953) (width 0.25) (layer B.Cu) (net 20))
 (segment (start 144.94 94.9953) (end 144.94 102) (width 0.25) (layer B.Cu) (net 20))
 (segment (start 144.94 102) (end 144.94 97.6242) (width 0.25) (layer F.Cu) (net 21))
 (segment (start 144.94 97.6242) (end 144.145 96.8292) (width 0.25) (layer F.Cu) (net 21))
 (segment (start 144.145 96.8292) (end 144.145 92.075) (width 0.25) (layer F.Cu) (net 21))
 (segment (start 142.4 102) (end 142.4 97.6242) (width 0.25) (layer B.Cu) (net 22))
 (segment (start 142.4 97.6242) (end 141.605 96.8292) (width 0.25) (layer B.Cu) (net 22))
 (segment (start 141.605 96.8292) (end 141.605 92.075) (width 0.25) (layer B.Cu) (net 22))
 (segment (start 139.065 92.075) (end 139.065 93.2503) (width 0.25) (layer F.Cu) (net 23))
 (segment (start 139.065 93.2503) (end 142.4 96.5853) (width 0.25) (layer F.Cu) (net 23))
 (segment (start 142.4 96.5853) (end 142.4 102) (width 0.25) (layer F.Cu) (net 23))
 (segment (start 136.525 92.075) (end 136.525 93.2503) (width 0.25) (layer B.Cu) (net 24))
 (segment (start 136.525 93.2503) (end 139.86 96.5853) (width 0.25) (layer B.Cu) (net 24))
 (segment (start 139.86 96.5853) (end 139.86 102) (width 0.25) (layer B.Cu) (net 24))
 (segment (start 139.86 102) (end 139.86 97.6242) (width 0.25) (layer F.Cu) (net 25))
 (segment (start 139.86 97.6242) (end 138.359 97.6242) (width 0.25) (layer F.Cu) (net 25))
 (segment (start 138.359 97.6242) (end 133.985 93.2503) (width 0.25) (layer F.Cu) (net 25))
 (segment (start 133.985 93.2503) (end 133.985 92.075) (width 0.25) (layer F.Cu) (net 25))
 (segment (start 137.32 102) (end 137.32 97.6242) (width 0.25) (layer B.Cu) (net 26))
 (segment (start 137.32 97.6242) (end 135.819 97.6242) (width 0.25) (layer B.Cu) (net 26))
 (segment (start 135.819 97.6242) (end 131.445 93.2503) (width 0.25) (layer B.Cu) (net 26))
 (segment (start 131.445 93.2503) (end 131.445 92.075) (width 0.25) (layer B.Cu) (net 26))
 (segment (start 137.32 102) (end 137.32 97.6242) (width 0.25) (layer F.Cu) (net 27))
 (segment (start 137.32 97.6242) (end 135.262 97.6242) (width 0.25) (layer F.Cu) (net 27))
 (segment (start 135.262 97.6242) (end 130.08 92.4424) (width 0.25) (layer F.Cu) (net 27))
 (segment (start 130.08 92.4424) (end 130.08 92.075) (width 0.25) (layer F.Cu) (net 27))
 (segment (start 130.08 92.075) (end 128.905 92.075) (width 0.25) (layer F.Cu) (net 27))
 (segment (start 134.78 102) (end 134.78 97.6242) (width 0.25) (layer B.Cu) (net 28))
 (segment (start 134.78 97.6242) (end 130.406 93.2503) (width 0.25) (layer B.Cu) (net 28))
 (segment (start 130.406 93.2503) (end 128.348 93.2503) (width 0.25) (layer B.Cu) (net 28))
 (segment (start 128.348 93.2503) (end 127.54 92.4424) (width 0.25) (layer B.Cu) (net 28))
 (segment (start 127.54 92.4424) (end 127.54 92.075) (width 0.25) (layer B.Cu) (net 28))
 (segment (start 127.54 92.075) (end 126.365 92.075) (width 0.25) (layer B.Cu) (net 28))
 (segment (start 175.42 102) (end 175.42 89.4931) (width 0.25) (layer F.Cu) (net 3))
 (segment (start 175.42 89.4931) (end 158.471 72.5445) (width 0.25) (layer F.Cu) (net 3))
 (segment (start 158.471 72.5445) (end 128.93 72.5445) (width 0.25) (layer F.Cu) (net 3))
 (segment (start 128.93 72.5445) (end 125 76.4739) (width 0.25) (layer F.Cu) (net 3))
 (segment (start 125 76.4739) (end 125 89.7244) (width 0.25) (layer F.Cu) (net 3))
 (segment (start 125 89.7244) (end 123.825 90.8997) (width 0.25) (layer F.Cu) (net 3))
 (segment (start 123.825 90.8997) (end 123.825 92.075) (width 0.25) (layer F.Cu) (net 3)))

